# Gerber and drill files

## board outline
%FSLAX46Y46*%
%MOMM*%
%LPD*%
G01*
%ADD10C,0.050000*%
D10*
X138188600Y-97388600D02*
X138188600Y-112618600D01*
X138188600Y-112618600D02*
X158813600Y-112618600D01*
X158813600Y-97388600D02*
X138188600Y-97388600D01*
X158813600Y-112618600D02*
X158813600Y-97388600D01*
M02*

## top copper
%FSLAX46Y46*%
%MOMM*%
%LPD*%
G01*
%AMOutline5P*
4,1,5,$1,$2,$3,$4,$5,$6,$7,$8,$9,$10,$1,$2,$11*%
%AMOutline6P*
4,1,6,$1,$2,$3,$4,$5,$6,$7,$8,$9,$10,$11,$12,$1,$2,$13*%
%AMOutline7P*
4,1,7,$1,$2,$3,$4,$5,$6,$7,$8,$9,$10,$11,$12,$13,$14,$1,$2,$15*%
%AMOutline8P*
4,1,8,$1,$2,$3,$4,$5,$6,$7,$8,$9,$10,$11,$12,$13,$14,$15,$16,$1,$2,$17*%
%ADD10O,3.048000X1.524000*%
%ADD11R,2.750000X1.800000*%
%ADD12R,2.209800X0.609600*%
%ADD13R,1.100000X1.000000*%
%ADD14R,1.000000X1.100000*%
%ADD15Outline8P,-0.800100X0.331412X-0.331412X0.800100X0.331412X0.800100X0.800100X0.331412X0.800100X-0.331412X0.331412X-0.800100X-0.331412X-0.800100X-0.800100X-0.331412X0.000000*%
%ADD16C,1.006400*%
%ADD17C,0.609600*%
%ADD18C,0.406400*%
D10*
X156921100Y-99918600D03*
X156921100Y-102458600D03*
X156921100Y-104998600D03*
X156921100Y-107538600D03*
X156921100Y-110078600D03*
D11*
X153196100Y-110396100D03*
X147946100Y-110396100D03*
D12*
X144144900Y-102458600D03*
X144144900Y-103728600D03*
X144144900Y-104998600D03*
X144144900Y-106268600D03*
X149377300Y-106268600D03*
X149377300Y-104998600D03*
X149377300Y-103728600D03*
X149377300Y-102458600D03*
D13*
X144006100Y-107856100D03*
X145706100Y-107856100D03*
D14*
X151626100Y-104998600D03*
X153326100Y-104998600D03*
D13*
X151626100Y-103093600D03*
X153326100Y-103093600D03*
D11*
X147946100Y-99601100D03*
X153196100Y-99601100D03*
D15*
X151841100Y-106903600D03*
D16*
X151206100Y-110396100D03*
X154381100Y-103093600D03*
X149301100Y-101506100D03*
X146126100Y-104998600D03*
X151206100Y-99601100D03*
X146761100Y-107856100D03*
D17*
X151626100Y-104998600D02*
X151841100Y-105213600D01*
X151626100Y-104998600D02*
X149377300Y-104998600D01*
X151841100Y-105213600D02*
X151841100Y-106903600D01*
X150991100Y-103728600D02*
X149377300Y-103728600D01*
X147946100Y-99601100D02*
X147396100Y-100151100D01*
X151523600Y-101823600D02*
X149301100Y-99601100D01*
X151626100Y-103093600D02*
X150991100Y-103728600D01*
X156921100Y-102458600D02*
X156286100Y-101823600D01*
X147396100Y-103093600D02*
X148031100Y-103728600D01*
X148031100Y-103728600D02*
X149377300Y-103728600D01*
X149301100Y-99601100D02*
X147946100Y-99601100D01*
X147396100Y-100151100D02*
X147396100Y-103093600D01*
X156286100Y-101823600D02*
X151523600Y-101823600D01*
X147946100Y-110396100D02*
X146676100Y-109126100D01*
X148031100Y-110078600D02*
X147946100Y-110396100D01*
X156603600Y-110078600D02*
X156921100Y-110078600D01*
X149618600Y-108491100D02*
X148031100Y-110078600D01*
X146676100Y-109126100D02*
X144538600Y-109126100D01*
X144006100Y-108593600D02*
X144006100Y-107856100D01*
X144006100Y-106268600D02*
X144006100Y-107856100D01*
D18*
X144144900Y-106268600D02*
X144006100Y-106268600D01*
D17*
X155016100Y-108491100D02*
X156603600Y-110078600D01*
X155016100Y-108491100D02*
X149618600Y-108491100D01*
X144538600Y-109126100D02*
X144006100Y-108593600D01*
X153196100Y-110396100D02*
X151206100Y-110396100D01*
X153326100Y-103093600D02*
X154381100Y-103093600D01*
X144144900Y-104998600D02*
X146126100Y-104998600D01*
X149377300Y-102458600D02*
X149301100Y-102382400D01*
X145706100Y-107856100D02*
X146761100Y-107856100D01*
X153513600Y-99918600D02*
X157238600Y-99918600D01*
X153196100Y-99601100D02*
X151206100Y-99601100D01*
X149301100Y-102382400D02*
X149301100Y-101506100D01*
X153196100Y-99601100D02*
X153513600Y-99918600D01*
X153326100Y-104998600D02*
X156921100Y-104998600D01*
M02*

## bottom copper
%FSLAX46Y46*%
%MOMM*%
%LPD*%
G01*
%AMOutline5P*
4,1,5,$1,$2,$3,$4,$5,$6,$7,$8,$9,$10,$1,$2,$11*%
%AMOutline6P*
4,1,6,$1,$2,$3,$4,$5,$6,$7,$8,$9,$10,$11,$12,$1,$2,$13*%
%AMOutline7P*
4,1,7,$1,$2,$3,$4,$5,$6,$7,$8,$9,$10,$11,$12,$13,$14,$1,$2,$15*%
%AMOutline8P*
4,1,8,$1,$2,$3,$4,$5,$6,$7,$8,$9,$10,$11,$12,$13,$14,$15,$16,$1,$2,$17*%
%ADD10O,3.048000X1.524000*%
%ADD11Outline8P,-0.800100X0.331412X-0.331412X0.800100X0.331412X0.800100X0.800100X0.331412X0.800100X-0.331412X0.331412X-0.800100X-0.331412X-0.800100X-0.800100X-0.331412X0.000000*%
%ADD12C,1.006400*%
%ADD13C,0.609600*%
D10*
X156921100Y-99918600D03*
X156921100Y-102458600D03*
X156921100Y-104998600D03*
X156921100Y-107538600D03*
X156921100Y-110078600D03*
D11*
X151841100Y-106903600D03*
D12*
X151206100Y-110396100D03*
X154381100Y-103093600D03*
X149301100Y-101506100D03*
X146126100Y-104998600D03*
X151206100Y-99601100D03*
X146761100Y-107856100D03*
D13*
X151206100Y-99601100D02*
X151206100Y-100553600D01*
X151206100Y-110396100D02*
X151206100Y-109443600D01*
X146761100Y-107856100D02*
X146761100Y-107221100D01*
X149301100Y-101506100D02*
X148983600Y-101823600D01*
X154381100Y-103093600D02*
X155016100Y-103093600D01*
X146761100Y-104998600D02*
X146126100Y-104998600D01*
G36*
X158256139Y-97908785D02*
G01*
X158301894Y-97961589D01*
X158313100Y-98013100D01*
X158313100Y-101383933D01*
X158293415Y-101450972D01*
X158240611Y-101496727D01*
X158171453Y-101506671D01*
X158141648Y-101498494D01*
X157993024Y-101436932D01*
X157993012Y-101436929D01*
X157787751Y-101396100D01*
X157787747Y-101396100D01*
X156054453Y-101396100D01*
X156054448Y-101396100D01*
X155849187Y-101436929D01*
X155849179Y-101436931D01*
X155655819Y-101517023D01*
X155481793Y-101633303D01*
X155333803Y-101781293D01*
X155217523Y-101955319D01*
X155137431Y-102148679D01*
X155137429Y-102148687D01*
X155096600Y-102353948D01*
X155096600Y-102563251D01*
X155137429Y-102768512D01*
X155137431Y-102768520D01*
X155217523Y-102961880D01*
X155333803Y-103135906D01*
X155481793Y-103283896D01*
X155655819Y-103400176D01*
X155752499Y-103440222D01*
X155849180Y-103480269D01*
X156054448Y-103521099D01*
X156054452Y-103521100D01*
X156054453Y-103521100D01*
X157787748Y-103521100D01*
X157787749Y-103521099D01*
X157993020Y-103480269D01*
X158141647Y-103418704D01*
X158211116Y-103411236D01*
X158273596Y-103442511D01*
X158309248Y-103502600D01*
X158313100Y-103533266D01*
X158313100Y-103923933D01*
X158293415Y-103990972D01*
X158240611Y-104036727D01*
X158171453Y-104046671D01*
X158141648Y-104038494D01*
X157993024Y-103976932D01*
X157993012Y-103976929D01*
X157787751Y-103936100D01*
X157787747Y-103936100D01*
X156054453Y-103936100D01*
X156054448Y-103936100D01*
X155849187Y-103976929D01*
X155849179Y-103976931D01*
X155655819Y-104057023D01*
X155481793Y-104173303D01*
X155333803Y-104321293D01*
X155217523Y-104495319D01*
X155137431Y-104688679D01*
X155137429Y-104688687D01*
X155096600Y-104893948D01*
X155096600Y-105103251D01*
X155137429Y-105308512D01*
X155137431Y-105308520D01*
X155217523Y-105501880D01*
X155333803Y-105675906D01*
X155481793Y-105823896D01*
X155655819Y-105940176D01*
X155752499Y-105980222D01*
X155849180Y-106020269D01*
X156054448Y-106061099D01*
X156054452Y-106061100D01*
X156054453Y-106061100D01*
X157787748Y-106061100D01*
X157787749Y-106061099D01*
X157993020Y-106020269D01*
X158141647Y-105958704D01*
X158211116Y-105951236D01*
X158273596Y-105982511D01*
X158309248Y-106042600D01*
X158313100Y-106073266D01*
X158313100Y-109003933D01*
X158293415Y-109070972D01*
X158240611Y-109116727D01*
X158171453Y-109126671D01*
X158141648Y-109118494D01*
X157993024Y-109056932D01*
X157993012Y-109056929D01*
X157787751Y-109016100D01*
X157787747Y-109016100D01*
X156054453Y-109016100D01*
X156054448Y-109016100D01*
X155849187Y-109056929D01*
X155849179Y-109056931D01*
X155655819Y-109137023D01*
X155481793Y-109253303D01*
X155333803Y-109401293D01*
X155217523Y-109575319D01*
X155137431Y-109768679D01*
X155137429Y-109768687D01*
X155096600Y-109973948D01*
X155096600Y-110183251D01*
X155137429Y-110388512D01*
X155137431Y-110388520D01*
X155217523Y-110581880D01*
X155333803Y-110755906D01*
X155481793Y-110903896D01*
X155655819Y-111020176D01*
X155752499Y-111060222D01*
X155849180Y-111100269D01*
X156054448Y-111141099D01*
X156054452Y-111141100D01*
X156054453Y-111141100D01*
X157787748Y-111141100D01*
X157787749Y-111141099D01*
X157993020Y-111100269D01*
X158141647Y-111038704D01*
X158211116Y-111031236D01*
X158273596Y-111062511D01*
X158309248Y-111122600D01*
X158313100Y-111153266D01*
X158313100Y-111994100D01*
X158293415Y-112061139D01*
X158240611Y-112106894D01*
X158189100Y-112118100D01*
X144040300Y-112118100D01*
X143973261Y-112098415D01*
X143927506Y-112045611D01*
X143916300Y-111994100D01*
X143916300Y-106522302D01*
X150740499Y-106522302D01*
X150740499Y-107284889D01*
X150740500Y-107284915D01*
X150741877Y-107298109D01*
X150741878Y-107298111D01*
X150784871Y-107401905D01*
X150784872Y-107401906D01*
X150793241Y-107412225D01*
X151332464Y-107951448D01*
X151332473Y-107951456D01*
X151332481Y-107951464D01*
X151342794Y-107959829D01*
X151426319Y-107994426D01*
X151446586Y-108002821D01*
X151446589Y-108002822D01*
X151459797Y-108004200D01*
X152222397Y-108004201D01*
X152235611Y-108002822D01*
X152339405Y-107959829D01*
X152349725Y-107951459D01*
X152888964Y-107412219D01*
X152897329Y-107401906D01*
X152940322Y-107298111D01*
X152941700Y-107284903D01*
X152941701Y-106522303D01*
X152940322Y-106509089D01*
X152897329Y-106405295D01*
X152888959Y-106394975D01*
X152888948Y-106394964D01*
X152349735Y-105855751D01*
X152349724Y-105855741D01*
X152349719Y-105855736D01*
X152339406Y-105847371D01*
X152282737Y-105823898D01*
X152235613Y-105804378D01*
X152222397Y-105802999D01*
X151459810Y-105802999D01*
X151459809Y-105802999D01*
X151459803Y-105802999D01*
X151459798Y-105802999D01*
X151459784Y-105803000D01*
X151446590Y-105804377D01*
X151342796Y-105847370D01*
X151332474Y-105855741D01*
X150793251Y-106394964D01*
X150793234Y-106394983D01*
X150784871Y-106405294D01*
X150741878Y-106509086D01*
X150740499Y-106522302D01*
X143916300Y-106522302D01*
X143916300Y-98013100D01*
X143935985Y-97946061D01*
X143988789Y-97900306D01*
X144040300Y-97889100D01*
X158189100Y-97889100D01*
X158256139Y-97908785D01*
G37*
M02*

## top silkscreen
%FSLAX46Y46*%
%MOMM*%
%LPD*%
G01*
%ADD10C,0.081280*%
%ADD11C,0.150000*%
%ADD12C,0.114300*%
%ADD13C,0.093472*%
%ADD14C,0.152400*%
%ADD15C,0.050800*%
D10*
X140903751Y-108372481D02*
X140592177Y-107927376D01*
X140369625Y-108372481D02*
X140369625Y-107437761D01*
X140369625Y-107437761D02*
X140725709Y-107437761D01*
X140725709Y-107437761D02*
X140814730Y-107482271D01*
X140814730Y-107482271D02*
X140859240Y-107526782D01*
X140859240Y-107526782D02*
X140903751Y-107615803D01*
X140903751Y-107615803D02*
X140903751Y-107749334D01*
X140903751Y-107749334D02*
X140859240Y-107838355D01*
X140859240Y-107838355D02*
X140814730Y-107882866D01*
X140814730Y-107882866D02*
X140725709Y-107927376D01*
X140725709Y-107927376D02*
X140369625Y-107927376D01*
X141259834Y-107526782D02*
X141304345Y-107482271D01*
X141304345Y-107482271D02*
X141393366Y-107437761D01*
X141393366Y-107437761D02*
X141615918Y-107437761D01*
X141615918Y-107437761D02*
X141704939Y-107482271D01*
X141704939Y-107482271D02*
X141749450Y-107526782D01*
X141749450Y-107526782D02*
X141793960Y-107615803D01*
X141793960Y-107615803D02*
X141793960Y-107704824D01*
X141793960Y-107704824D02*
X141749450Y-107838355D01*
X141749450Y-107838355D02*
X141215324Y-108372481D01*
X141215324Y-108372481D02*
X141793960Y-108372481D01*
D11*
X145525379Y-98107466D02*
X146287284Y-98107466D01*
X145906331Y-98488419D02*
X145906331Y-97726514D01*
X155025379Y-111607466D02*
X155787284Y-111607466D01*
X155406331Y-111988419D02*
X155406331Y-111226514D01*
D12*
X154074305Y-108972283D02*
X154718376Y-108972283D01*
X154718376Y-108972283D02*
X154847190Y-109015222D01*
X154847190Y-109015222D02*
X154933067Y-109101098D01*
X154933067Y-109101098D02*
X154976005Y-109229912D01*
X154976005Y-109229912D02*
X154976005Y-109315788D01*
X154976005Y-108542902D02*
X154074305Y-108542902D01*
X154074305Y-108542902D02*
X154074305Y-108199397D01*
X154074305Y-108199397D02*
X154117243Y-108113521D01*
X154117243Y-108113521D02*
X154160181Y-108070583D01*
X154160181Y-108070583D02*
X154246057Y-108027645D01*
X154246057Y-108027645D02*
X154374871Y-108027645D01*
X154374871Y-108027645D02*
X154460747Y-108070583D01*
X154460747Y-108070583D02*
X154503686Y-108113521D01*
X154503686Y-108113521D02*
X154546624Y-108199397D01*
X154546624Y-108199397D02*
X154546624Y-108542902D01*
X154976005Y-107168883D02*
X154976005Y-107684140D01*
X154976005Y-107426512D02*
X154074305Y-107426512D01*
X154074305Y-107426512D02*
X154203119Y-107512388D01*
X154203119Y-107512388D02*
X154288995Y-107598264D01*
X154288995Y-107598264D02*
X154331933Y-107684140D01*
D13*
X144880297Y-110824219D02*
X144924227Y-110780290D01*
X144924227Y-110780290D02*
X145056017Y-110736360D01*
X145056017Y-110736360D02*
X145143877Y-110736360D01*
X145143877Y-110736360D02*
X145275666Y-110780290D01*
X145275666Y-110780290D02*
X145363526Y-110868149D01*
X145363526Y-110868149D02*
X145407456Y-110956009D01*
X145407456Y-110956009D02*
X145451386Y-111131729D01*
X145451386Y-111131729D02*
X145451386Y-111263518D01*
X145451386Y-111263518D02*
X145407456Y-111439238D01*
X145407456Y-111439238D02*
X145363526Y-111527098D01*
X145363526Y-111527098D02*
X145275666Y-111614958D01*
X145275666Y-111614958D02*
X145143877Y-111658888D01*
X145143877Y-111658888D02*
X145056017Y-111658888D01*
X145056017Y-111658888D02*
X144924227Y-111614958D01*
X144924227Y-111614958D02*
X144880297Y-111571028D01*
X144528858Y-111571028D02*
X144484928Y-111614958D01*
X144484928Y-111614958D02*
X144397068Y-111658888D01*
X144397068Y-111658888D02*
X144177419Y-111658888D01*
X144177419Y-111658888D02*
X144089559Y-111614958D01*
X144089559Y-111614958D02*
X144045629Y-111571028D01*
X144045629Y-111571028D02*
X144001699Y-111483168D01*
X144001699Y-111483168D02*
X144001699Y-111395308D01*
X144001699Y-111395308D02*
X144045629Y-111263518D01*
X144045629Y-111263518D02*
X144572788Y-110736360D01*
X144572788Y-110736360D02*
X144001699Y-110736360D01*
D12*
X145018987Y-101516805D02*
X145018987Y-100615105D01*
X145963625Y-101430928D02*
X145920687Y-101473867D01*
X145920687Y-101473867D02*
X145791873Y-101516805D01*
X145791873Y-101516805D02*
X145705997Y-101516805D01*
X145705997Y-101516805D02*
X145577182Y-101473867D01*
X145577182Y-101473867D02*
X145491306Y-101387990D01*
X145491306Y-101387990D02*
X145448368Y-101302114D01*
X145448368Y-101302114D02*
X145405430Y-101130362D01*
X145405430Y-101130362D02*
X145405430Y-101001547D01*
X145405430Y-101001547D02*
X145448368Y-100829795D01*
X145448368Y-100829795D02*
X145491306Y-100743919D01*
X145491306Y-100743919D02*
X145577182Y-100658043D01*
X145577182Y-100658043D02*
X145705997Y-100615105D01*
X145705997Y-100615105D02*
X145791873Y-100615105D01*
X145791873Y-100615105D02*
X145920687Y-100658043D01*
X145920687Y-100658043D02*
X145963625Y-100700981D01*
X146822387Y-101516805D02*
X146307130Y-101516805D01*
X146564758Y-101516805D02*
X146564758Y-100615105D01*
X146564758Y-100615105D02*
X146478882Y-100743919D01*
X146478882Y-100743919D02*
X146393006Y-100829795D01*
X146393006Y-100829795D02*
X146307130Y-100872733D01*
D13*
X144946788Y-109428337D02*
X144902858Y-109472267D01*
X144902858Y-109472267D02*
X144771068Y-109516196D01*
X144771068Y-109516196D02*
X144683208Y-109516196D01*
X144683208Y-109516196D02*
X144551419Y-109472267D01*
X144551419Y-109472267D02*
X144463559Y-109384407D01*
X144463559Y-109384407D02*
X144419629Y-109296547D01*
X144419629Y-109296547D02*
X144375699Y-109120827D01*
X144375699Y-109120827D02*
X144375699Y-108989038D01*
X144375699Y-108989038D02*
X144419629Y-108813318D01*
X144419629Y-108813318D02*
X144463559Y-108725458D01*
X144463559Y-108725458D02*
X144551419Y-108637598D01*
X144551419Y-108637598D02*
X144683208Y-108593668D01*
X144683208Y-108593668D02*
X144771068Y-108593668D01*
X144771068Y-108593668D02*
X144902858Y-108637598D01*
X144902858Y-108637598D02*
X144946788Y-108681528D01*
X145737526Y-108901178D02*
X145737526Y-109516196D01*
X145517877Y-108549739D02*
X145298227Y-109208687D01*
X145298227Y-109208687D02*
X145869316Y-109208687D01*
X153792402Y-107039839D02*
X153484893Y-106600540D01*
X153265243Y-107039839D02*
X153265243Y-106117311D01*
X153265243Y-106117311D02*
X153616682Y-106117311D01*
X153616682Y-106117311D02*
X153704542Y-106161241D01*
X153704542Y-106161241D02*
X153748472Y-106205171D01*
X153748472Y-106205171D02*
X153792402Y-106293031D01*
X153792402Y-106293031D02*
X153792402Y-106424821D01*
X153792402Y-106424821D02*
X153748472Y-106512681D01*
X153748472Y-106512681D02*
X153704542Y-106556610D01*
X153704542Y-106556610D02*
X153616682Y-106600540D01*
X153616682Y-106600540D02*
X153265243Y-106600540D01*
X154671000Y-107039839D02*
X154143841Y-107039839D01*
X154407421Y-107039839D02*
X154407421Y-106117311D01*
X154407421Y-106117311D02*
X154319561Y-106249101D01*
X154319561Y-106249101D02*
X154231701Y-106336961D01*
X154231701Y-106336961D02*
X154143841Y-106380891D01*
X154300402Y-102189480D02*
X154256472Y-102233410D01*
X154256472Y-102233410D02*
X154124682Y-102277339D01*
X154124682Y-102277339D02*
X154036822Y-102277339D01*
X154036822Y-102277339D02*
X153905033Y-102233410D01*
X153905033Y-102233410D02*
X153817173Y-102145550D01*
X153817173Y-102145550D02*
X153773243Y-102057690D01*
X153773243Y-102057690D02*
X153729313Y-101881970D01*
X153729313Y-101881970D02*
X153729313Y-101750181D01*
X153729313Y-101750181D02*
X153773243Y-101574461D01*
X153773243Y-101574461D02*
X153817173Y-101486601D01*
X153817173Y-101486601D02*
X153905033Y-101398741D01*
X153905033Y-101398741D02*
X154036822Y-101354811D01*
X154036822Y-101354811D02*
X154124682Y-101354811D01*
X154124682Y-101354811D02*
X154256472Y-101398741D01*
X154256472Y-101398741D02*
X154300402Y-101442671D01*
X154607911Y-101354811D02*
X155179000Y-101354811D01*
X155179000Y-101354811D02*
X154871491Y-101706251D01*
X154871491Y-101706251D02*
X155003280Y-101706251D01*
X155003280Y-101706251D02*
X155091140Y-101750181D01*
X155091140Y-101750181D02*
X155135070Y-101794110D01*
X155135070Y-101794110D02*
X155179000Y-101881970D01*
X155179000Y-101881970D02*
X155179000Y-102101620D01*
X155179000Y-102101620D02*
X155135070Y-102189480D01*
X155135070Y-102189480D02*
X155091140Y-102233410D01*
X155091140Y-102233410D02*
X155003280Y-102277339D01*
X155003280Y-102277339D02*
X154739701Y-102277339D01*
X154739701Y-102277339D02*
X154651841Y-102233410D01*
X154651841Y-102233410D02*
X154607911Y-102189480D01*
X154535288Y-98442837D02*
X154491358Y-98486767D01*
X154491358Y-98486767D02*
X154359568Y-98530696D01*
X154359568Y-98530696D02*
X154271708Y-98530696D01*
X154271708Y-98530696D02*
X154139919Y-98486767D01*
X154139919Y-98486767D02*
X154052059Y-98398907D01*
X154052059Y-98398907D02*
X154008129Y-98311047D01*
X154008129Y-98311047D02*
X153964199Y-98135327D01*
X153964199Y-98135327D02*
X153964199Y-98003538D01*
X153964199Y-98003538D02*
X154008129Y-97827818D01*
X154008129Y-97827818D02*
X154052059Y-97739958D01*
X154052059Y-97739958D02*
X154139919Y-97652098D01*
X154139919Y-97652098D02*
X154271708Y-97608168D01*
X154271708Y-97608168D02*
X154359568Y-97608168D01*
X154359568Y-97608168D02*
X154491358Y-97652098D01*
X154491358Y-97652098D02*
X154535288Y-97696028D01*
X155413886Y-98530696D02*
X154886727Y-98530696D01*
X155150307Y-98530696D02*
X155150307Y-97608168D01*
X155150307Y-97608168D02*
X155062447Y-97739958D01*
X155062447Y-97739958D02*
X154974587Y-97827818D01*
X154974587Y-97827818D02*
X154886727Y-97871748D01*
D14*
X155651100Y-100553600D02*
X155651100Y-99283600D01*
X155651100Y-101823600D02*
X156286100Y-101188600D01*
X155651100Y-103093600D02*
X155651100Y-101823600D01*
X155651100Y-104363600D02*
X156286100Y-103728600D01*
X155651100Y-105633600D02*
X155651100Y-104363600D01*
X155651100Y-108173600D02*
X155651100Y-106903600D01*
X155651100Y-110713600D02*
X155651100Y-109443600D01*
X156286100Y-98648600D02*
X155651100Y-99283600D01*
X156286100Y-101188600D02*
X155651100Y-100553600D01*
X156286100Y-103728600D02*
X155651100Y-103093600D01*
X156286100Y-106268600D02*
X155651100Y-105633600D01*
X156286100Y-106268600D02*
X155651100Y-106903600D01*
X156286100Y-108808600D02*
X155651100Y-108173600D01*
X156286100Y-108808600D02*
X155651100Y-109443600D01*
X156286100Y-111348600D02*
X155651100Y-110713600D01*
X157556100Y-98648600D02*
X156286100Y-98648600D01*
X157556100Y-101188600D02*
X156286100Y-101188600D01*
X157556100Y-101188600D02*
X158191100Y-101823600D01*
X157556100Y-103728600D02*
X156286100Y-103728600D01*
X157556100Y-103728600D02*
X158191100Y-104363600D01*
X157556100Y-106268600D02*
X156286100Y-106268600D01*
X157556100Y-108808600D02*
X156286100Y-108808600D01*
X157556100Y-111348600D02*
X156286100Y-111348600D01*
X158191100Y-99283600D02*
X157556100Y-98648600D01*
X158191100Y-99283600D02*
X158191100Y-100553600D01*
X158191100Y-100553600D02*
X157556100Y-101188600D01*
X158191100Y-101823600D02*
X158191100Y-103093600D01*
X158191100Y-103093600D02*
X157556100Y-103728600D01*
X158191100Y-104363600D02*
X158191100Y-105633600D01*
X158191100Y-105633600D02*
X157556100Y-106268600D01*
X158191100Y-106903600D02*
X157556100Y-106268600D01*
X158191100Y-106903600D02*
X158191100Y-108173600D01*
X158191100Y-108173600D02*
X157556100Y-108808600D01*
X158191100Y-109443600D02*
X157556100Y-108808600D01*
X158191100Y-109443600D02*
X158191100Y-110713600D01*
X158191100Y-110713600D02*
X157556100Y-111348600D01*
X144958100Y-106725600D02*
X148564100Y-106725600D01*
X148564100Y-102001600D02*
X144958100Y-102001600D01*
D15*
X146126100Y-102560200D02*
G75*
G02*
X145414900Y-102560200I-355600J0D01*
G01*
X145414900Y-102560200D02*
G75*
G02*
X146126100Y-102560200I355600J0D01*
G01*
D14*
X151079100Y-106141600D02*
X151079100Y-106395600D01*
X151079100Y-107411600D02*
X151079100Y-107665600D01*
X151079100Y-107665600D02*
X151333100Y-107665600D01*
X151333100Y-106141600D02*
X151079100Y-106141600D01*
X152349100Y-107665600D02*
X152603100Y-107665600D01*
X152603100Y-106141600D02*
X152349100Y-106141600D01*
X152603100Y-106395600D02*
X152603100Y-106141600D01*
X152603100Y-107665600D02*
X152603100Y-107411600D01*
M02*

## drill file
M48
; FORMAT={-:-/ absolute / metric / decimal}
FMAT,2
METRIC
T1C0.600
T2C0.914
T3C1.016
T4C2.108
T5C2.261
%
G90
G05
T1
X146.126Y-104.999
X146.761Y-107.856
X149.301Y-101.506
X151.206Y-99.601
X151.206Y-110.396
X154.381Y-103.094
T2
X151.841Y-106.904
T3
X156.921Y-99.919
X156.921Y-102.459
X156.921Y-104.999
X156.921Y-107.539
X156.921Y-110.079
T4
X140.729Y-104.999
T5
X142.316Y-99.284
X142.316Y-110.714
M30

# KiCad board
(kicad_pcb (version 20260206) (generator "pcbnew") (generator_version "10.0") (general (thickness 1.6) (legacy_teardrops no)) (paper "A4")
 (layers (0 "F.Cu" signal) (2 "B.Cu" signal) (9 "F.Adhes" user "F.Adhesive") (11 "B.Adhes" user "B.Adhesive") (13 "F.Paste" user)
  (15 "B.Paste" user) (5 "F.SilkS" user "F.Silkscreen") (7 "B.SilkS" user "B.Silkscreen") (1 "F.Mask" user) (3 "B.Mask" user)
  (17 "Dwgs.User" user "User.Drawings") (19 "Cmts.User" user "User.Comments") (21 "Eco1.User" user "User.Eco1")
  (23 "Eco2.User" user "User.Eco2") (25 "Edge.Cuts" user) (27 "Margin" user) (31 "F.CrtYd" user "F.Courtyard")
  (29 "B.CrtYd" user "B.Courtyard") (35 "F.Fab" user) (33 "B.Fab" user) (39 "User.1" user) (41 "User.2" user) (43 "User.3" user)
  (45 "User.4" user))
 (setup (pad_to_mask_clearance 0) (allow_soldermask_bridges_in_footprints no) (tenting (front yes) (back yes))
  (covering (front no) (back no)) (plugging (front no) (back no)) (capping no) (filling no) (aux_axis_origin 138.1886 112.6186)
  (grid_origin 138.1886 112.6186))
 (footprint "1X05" (layer "F.Cu") (at 156.9211 104.9986 -90)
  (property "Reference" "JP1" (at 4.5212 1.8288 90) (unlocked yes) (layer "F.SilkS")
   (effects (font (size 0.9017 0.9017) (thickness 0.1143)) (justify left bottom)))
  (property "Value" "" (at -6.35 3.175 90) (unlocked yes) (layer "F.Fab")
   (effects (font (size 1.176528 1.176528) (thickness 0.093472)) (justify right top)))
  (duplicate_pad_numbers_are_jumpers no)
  (fp_line (start -4.445 1.27) (end -5.715 1.27) (stroke (width 0.1524) (type solid)) (layer "F.SilkS"))
  (fp_line (start -3.175 1.27) (end -3.81 0.635) (stroke (width 0.1524) (type solid)) (layer "F.SilkS"))
  (fp_line (start -1.905 1.27) (end -3.175 1.27) (stroke (width 0.1524) (type solid)) (layer "F.SilkS"))
  (fp_line (start -0.635 1.27) (end -1.27 0.635) (stroke (width 0.1524) (type solid)) (layer "F.SilkS"))
  (fp_line (start 0.635 1.27) (end -0.635 1.27) (stroke (width 0.1524) (type solid)) (layer "F.SilkS"))
  (fp_line (start 3.175 1.27) (end 1.905 1.27) (stroke (width 0.1524) (type solid)) (layer "F.SilkS"))
  (fp_line (start 5.715 1.27) (end 4.445 1.27) (stroke (width 0.1524) (type solid)) (layer "F.SilkS"))
  (fp_line (start -6.35 0.635) (end -5.715 1.27) (stroke (width 0.1524) (type solid)) (layer "F.SilkS"))
  (fp_line (start -3.81 0.635) (end -4.445 1.27) (stroke (width 0.1524) (type solid)) (layer "F.SilkS"))
  (fp_line (start -1.27 0.635) (end -1.905 1.27) (stroke (width 0.1524) (type solid)) (layer "F.SilkS"))
  (fp_line (start 1.27 0.635) (end 0.635 1.27) (stroke (width 0.1524) (type solid)) (layer "F.SilkS"))
  (fp_line (start 1.27 0.635) (end 1.905 1.27) (stroke (width 0.1524) (type solid)) (layer "F.SilkS"))
  (fp_line (start 3.81 0.635) (end 3.175 1.27) (stroke (width 0.1524) (type solid)) (layer "F.SilkS"))
  (fp_line (start 3.81 0.635) (end 4.445 1.27) (stroke (width 0.1524) (type solid)) (layer "F.SilkS"))
  (fp_line (start 6.35 0.635) (end 5.715 1.27) (stroke (width 0.1524) (type solid)) (layer "F.SilkS"))
  (fp_line (start -6.35 -0.635) (end -6.35 0.635) (stroke (width 0.1524) (type solid)) (layer "F.SilkS"))
  (fp_line (start -3.81 -0.635) (end -3.81 0.635) (stroke (width 0.1524) (type solid)) (layer "F.SilkS"))
  (fp_line (start -3.81 -0.635) (end -3.175 -1.27) (stroke (width 0.1524) (type solid)) (layer "F.SilkS"))
  (fp_line (start -1.27 -0.635) (end -1.27 0.635) (stroke (width 0.1524) (type solid)) (layer "F.SilkS"))
  (fp_line (start -1.27 -0.635) (end -0.635 -1.27) (stroke (width 0.1524) (type solid)) (layer "F.SilkS"))
  (fp_line (start 1.27 -0.635) (end 1.27 0.635) (stroke (width 0.1524) (type solid)) (layer "F.SilkS"))
  (fp_line (start 3.81 -0.635) (end 3.81 0.635) (stroke (width 0.1524) (type solid)) (layer "F.SilkS"))
  (fp_line (start 6.35 -0.635) (end 6.35 0.635) (stroke (width 0.1524) (type solid)) (layer "F.SilkS"))
  (fp_line (start -5.715 -1.27) (end -6.35 -0.635) (stroke (width 0.1524) (type solid)) (layer "F.SilkS"))
  (fp_line (start -5.715 -1.27) (end -4.445 -1.27) (stroke (width 0.1524) (type solid)) (layer "F.SilkS"))
  (fp_line (start -4.445 -1.27) (end -3.81 -0.635) (stroke (width 0.1524) (type solid)) (layer "F.SilkS"))
  (fp_line (start -3.175 -1.27) (end -1.905 -1.27) (stroke (width 0.1524) (type solid)) (layer "F.SilkS"))
  (fp_line (start -1.905 -1.27) (end -1.27 -0.635) (stroke (width 0.1524) (type solid)) (layer "F.SilkS"))
  (fp_line (start -0.635 -1.27) (end 0.635 -1.27) (stroke (width 0.1524) (type solid)) (layer "F.SilkS"))
  (fp_line (start 0.635 -1.27) (end 1.27 -0.635) (stroke (width 0.1524) (type solid)) (layer "F.SilkS"))
  (fp_line (start 1.905 -1.27) (end 1.27 -0.635) (stroke (width 0.1524) (type solid)) (layer "F.SilkS"))
  (fp_line (start 1.905 -1.27) (end 3.175 -1.27) (stroke (width 0.1524) (type solid)) (layer "F.SilkS"))
  (fp_line (start 3.175 -1.27) (end 3.81 -0.635) (stroke (width 0.1524) (type solid)) (layer "F.SilkS"))
  (fp_line (start 4.445 -1.27) (end 3.81 -0.635) (stroke (width 0.1524) (type solid)) (layer "F.SilkS"))
  (fp_line (start 4.445 -1.27) (end 5.715 -1.27) (stroke (width 0.1524) (type solid)) (layer "F.SilkS"))
  (fp_line (start 5.715 -1.27) (end 6.35 -0.635) (stroke (width 0.1524) (type solid)) (layer "F.SilkS"))
  (pad "1" thru_hole oval (at -5.08 0) (size 3.048 1.524) (drill 1.016) (layers "*.Cu" "*.Mask") (remove_unused_layers no) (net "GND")
   (solder_mask_margin 0.1016) (zone_connect 2) (thermal_bridge_angle 0))
  (pad "2" thru_hole oval (at -2.54 0) (size 3.048 1.524) (drill 1.016) (layers "*.Cu" "*.Mask") (remove_unused_layers no) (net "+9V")
   (solder_mask_margin 0.1016) (thermal_bridge_angle 0))
  (pad "3" thru_hole oval (at 0 0) (size 3.048 1.524) (drill 1.016) (layers "*.Cu" "*.Mask") (remove_unused_layers no) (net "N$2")
   (solder_mask_margin 0.1016) (thermal_bridge_angle 0))
  (pad "4" thru_hole oval (at 2.54 0) (size 3.048 1.524) (drill 1.016) (layers "*.Cu" "*.Mask") (remove_unused_layers no) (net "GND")
   (solder_mask_margin 0.1016) (zone_connect 2) (thermal_bridge_angle 0))
  (pad "5" thru_hole oval (at 5.08 0) (size 3.048 1.524) (drill 1.016) (layers "*.Cu" "*.Mask") (remove_unused_layers no) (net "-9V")
   (solder_mask_margin 0.1016) (thermal_bridge_angle 0)))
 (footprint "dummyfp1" (layer "F.Cu") (at 142.3161 110.7136)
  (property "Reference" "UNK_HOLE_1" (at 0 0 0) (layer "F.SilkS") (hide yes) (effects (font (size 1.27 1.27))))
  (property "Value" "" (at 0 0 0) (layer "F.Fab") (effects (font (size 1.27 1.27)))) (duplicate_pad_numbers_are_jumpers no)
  (pad "" np_thru_hole circle (at 0 0) (size 2.2606 2.2606) (drill 2.2606) (layers "*.Cu" "*.Mask")))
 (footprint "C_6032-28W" (layer "F.Cu") (at 150.5711 110.3961)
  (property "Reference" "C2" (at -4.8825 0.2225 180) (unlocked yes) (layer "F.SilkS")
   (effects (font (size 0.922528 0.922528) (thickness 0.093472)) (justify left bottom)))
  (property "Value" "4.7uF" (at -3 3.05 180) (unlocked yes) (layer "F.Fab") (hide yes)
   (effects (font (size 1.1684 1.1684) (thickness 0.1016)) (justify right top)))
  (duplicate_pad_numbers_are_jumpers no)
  (pad "+" smd rect (at 2.625 0) (size 2.75 1.8) (layers "F.Cu" "F.Mask" "F.Paste") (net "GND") (solder_mask_margin 0.1016)
   (solder_paste_margin 0) (thermal_bridge_angle 0))
  (pad "-" smd rect (at -2.625 0) (size 2.75 1.8) (layers "F.Cu" "F.Mask" "F.Paste") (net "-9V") (solder_mask_margin 0.1016)
   (solder_paste_margin 0) (thermal_bridge_angle 0)))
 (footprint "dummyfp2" (layer "F.Cu") (at 142.3161 99.2836)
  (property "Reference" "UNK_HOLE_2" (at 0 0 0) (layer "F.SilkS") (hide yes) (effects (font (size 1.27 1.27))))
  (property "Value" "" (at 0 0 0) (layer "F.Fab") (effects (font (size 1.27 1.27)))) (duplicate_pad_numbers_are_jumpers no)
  (pad "" np_thru_hole circle (at 0 0) (size 2.2606 2.2606) (drill 2.2606) (layers "*.Cu" "*.Mask")))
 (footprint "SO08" (layer "F.Cu") (at 146.7611 104.3636 -90)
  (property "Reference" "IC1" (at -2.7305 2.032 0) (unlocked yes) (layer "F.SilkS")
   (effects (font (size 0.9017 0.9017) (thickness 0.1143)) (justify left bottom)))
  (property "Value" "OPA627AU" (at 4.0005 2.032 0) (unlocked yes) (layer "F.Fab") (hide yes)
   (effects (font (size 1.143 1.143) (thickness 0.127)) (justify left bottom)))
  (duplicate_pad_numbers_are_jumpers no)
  (fp_line (start 2.362 1.803) (end 2.362 -1.803) (stroke (width 0.1524) (type solid)) (layer "F.SilkS"))
  (fp_line (start -2.362 -1.803) (end -2.362 1.803) (stroke (width 0.1524) (type solid)) (layer "F.SilkS"))
  (fp_circle (center -1.8034 0.9906) (end -1.4478 0.9906) (stroke (width 0.0508) (type solid)) (fill no) (layer "F.SilkS"))
  (pad "1" smd rect (at -1.905 2.6162 270) (size 0.6096 2.2098) (layers "F.Cu" "F.Mask" "F.Paste") (solder_mask_margin 0.1016)
   (solder_paste_margin 0) (thermal_bridge_angle 0))
  (pad "2" smd rect (at -0.635 2.6162 270) (size 0.6096 2.2098) (layers "F.Cu" "F.Mask" "F.Paste") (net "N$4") (solder_mask_margin 0.1016)
   (solder_paste_margin 0) (thermal_bridge_angle 0))
  (pad "3" smd rect (at 0.635 2.6162 270) (size 0.6096 2.2098) (layers "F.Cu" "F.Mask" "F.Paste") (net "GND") (solder_mask_margin 0.1016)
   (solder_paste_margin 0) (thermal_bridge_angle 0))
  (pad "4" smd rect (at 1.905 2.6162 270) (size 0.6096 2.2098) (layers "F.Cu" "F.Mask" "F.Paste") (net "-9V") (solder_mask_margin 0.1016)
   (solder_paste_margin 0) (thermal_bridge_angle 0))
  (pad "5" smd rect (at 1.905 -2.6162 270) (size 0.6096 2.2098) (layers "F.Cu" "F.Mask" "F.Paste") (solder_mask_margin 0.1016)
   (solder_paste_margin 0) (thermal_bridge_angle 0))
  (pad "6" smd rect (at 0.635 -2.6162 270) (size 0.6096 2.2098) (layers "F.Cu" "F.Mask" "F.Paste") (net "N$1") (solder_mask_margin 0.1016)
   (solder_paste_margin 0) (thermal_bridge_angle 0))
  (pad "7" smd rect (at -0.635 -2.6162 270) (size 0.6096 2.2098) (layers "F.Cu" "F.Mask" "F.Paste") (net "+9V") (solder_mask_margin 0.1016)
   (solder_paste_margin 0) (thermal_bridge_angle 0))
  (pad "8" smd rect (at -1.905 -2.6162 270) (size 0.6096 2.2098) (layers "F.Cu" "F.Mask" "F.Paste") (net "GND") (solder_mask_margin 0.1016)
   (solder_paste_margin 0) (thermal_bridge_angle 0)))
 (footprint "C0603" (layer "F.Cu") (at 144.8561 107.8561)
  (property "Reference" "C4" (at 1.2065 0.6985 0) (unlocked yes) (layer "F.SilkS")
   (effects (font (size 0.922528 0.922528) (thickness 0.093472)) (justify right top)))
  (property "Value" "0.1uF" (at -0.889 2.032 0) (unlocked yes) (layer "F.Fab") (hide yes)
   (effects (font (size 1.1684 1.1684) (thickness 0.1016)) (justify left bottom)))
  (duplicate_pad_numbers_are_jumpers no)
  (pad "1" smd rect (at -0.85 0) (size 1.1 1) (layers "F.Cu" "F.Mask" "F.Paste") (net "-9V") (solder_mask_margin 0.1016)
   (solder_paste_margin 0) (thermal_bridge_angle 0))
  (pad "2" smd rect (at 0.85 0) (size 1.1 1) (layers "F.Cu" "F.Mask" "F.Paste") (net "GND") (solder_mask_margin 0.1016)
   (solder_paste_margin 0) (thermal_bridge_angle 0)))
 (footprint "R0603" (layer "F.Cu") (at 152.4761 104.9986)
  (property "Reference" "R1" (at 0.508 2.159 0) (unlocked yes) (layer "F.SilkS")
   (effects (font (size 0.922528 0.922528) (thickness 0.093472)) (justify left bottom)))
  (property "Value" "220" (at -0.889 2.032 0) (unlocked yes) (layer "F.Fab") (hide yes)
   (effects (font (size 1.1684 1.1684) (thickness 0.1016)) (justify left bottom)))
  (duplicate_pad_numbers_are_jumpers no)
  (pad "1" smd rect (at -0.85 0) (size 1 1.1) (layers "F.Cu" "F.Mask" "F.Paste") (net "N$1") (solder_mask_margin 0.1016)
   (solder_paste_margin 0) (thermal_bridge_angle 0))
  (pad "2" smd rect (at 0.85 0) (size 1 1.1) (layers "F.Cu" "F.Mask" "F.Paste") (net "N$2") (solder_mask_margin 0.1016)
   (solder_paste_margin 0) (thermal_bridge_angle 0)))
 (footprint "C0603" (layer "F.Cu") (at 152.4761 103.0936)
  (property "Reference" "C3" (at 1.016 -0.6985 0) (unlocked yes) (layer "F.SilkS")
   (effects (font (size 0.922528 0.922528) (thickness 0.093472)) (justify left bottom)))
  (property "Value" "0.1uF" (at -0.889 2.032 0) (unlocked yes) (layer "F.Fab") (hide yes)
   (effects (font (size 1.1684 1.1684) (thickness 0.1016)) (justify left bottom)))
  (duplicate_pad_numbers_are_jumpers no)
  (pad "1" smd rect (at -0.85 0) (size 1.1 1) (layers "F.Cu" "F.Mask" "F.Paste") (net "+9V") (solder_mask_margin 0.1016)
   (solder_paste_margin 0) (thermal_bridge_angle 0))
  (pad "2" smd rect (at 0.85 0) (size 1.1 1) (layers "F.Cu" "F.Mask" "F.Paste") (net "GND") (solder_mask_margin 0.1016)
   (solder_paste_margin 0) (thermal_bridge_angle 0)))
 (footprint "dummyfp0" (layer "F.Cu") (at 140.7286 104.9986)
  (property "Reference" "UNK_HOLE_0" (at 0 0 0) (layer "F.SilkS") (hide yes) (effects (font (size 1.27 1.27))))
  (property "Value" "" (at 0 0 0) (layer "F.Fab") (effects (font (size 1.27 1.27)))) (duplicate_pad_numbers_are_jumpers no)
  (pad "" np_thru_hole circle (at 0 0) (size 2.1082 2.1082) (drill 2.1082) (layers "*.Cu" "*.Mask")))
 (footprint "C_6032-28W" (layer "F.Cu") (at 150.5711 99.6011 180)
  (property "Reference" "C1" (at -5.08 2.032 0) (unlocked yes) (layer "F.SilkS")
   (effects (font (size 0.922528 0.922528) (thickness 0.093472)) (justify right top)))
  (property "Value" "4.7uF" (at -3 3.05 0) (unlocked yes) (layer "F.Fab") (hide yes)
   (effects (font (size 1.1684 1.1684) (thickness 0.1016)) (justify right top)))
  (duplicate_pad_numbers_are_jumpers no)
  (pad "+" smd rect (at 2.625 0 180) (size 2.75 1.8) (layers "F.Cu" "F.Mask" "F.Paste") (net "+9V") (solder_mask_margin 0.1016)
   (solder_paste_margin 0) (thermal_bridge_angle 0))
  (pad "-" smd rect (at -2.625 0 180) (size 2.75 1.8) (layers "F.Cu" "F.Mask" "F.Paste") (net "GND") (solder_mask_margin 0.1016)
   (solder_paste_margin 0) (thermal_bridge_angle 0)))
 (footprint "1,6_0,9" (layer "F.Cu") (at 151.8411 106.9036)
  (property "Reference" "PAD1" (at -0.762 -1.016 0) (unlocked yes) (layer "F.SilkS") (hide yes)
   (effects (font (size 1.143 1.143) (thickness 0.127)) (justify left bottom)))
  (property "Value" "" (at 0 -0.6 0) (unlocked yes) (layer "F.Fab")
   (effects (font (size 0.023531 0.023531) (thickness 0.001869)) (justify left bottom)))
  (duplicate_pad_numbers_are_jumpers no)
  (fp_line (start -0.762 -0.762) (end -0.762 -0.508) (stroke (width 0.1524) (type solid)) (layer "F.SilkS"))
  (fp_line (start -0.762 0.508) (end -0.762 0.762) (stroke (width 0.1524) (type solid)) (layer "F.SilkS"))
  (fp_line (start -0.762 0.762) (end -0.508 0.762) (stroke (width 0.1524) (type solid)) (layer "F.SilkS"))
  (fp_line (start -0.508 -0.762) (end -0.762 -0.762) (stroke (width 0.1524) (type solid)) (layer "F.SilkS"))
  (fp_line (start 0.508 0.762) (end 0.762 0.762) (stroke (width 0.1524) (type solid)) (layer "F.SilkS"))
  (fp_line (start 0.762 -0.762) (end 0.508 -0.762) (stroke (width 0.1524) (type solid)) (layer "F.SilkS"))
  (fp_line (start 0.762 -0.508) (end 0.762 -0.762) (stroke (width 0.1524) (type solid)) (layer "F.SilkS"))
  (fp_line (start 0.762 0.762) (end 0.762 0.508) (stroke (width 0.1524) (type solid)) (layer "F.SilkS"))
  (pad "1" thru_hole roundrect (at 0 0) (size 1.6002 1.6002) (drill 0.9144) (layers "*.Cu" "*.Mask") (remove_unused_layers no)
   (roundrect_rratio 0.25) (chamfer_ratio 0.2928932188) (chamfer top_left top_right bottom_left bottom_right) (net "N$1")
   (solder_mask_margin 0.1016) (thermal_bridge_angle 0)))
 (gr_line (start 138.1886 97.3886) (end 138.1886 112.6186) (stroke (width 0.05) (type solid)) (layer "Edge.Cuts"))
 (gr_line (start 138.1886 112.6186) (end 158.8136 112.6186) (stroke (width 0.05) (type solid)) (layer "Edge.Cuts"))
 (gr_line (start 158.8136 97.3886) (end 138.1886 97.3886) (stroke (width 0.05) (type solid)) (layer "Edge.Cuts"))
 (gr_line (start 158.8136 112.6186) (end 158.8136 97.3886) (stroke (width 0.05) (type solid)) (layer "Edge.Cuts"))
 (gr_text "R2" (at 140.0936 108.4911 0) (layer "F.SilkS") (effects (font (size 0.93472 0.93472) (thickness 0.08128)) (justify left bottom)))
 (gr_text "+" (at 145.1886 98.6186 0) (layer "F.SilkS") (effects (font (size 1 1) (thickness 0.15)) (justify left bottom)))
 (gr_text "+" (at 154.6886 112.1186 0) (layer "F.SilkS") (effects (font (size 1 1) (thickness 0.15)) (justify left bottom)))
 (segment (start 151.6261 104.9986) (end 151.8411 105.2136) (width 0.6096) (layer "F.Cu") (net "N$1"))
 (segment (start 151.6261 104.9986) (end 149.3773 104.9986) (width 0.6096) (layer "F.Cu") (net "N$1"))
 (segment (start 151.8411 105.2136) (end 151.8411 106.9036) (width 0.6096) (layer "F.Cu") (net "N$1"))
 (segment (start 150.9911 103.7286) (end 149.3773 103.7286) (width 0.6096) (layer "F.Cu") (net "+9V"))
 (segment (start 147.9461 99.6011) (end 147.3961 100.1511) (width 0.6096) (layer "F.Cu") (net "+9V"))
 (segment (start 151.5236 101.8236) (end 149.3011 99.6011) (width 0.6096) (layer "F.Cu") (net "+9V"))
 (segment (start 151.6261 103.0936) (end 150.9911 103.7286) (width 0.6096) (layer "F.Cu") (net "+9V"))
 (segment (start 156.9211 102.4586) (end 156.2861 101.8236) (width 0.6096) (layer "F.Cu") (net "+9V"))
 (segment (start 147.3961 103.0936) (end 148.0311 103.7286) (width 0.6096) (layer "F.Cu") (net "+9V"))
 (segment (start 148.0311 103.7286) (end 149.3773 103.7286) (width 0.6096) (layer "F.Cu") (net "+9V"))
 (segment (start 149.3011 99.6011) (end 147.9461 99.6011) (width 0.6096) (layer "F.Cu") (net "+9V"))
 (segment (start 147.3961 100.1511) (end 147.3961 103.0936) (width 0.6096) (layer "F.Cu") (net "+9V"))
 (segment (start 156.2861 101.8236) (end 151.5236 101.8236) (width 0.6096) (layer "F.Cu") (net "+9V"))
 (segment (start 147.9461 110.3961) (end 146.6761 109.1261) (width 0.6096) (layer "F.Cu") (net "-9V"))
 (segment (start 148.0311 110.0786) (end 147.9461 110.3961) (width 0.6096) (layer "F.Cu") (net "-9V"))
 (segment (start 156.6036 110.0786) (end 156.9211 110.0786) (width 0.6096) (layer "F.Cu") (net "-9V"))
 (segment (start 149.6186 108.4911) (end 148.0311 110.0786) (width 0.6096) (layer "F.Cu") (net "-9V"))
 (segment (start 146.6761 109.1261) (end 144.5386 109.1261) (width 0.6096) (layer "F.Cu") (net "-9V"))
 (segment (start 144.0061 108.5936) (end 144.0061 107.8561) (width 0.6096) (layer "F.Cu") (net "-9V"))
 (segment (start 144.0061 106.2686) (end 144.0061 107.8561) (width 0.6096) (layer "F.Cu") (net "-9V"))
 (segment (start 144.1449 106.2686) (end 144.0061 106.2686) (width 0.4064) (layer "F.Cu") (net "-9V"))
 (segment (start 155.0161 108.4911) (end 156.6036 110.0786) (width 0.6096) (layer "F.Cu") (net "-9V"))
 (segment (start 155.0161 108.4911) (end 149.6186 108.4911) (width 0.6096) (layer "F.Cu") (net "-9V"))
 (segment (start 144.5386 109.1261) (end 144.0061 108.5936) (width 0.6096) (layer "F.Cu") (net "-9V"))
 (segment (start 153.1961 110.3961) (end 151.2061 110.3961) (width 0.6096) (layer "F.Cu") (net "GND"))
 (segment (start 153.3261 103.0936) (end 154.3811 103.0936) (width 0.6096) (layer "F.Cu") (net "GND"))
 (segment (start 144.1449 104.9986) (end 146.1261 104.9986) (width 0.6096) (layer "F.Cu") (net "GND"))
 (segment (start 149.3773 102.4586) (end 149.3011 102.3824) (width 0.6096) (layer "F.Cu") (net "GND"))
 (segment (start 145.7061 107.8561) (end 146.7611 107.8561) (width 0.6096) (layer "F.Cu") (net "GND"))
 (segment (start 153.5136 99.9186) (end 157.2386 99.9186) (width 0.6096) (layer "F.Cu") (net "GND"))
 (segment (start 153.1961 99.6011) (end 151.2061 99.6011) (width 0.6096) (layer "F.Cu") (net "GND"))
 (segment (start 149.3011 102.3824) (end 149.3011 101.5061) (width 0.6096) (layer "F.Cu") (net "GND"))
 (segment (start 153.1961 99.6011) (end 153.5136 99.9186) (width 0.6096) (layer "F.Cu") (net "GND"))
 (via (at 151.2061 110.3961) (size 1.0064) (drill 0.6) (layers "F.Cu" "B.Cu") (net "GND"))
 (via (at 154.3811 103.0936) (size 1.0064) (drill 0.6) (layers "F.Cu" "B.Cu") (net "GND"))
 (via (at 149.3011 101.5061) (size 1.0064) (drill 0.6) (layers "F.Cu" "B.Cu") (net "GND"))
 (via (at 146.1261 104.9986) (size 1.0064) (drill 0.6) (layers "F.Cu" "B.Cu") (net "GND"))
 (via (at 151.2061 99.6011) (size 1.0064) (drill 0.6) (layers "F.Cu" "B.Cu") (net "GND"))
 (via (at 146.7611 107.8561) (size 1.0064) (drill 0.6) (layers "F.Cu" "B.Cu") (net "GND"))
 (segment (start 151.2061 99.6011) (end 151.2061 100.5536) (width 0.6096) (layer "B.Cu") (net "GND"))
 (segment (start 151.2061 110.3961) (end 151.2061 109.4436) (width 0.6096) (layer "B.Cu") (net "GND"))
 (segment (start 146.7611 107.8561) (end 146.7611 107.2211) (width 0.6096) (layer "B.Cu") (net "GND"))
 (segment (start 149.3011 101.5061) (end 148.9836 101.8236) (width 0.6096) (layer "B.Cu") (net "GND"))
 (segment (start 154.3811 103.0936) (end 155.0161 103.0936) (width 0.6096) (layer "B.Cu") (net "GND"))
 (segment (start 146.7611 104.9986) (end 146.1261 104.9986) (width 0.6096) (layer "B.Cu") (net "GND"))
 (segment (start 153.3261 104.9986) (end 156.9211 104.9986) (width 0.6096) (layer "F.Cu") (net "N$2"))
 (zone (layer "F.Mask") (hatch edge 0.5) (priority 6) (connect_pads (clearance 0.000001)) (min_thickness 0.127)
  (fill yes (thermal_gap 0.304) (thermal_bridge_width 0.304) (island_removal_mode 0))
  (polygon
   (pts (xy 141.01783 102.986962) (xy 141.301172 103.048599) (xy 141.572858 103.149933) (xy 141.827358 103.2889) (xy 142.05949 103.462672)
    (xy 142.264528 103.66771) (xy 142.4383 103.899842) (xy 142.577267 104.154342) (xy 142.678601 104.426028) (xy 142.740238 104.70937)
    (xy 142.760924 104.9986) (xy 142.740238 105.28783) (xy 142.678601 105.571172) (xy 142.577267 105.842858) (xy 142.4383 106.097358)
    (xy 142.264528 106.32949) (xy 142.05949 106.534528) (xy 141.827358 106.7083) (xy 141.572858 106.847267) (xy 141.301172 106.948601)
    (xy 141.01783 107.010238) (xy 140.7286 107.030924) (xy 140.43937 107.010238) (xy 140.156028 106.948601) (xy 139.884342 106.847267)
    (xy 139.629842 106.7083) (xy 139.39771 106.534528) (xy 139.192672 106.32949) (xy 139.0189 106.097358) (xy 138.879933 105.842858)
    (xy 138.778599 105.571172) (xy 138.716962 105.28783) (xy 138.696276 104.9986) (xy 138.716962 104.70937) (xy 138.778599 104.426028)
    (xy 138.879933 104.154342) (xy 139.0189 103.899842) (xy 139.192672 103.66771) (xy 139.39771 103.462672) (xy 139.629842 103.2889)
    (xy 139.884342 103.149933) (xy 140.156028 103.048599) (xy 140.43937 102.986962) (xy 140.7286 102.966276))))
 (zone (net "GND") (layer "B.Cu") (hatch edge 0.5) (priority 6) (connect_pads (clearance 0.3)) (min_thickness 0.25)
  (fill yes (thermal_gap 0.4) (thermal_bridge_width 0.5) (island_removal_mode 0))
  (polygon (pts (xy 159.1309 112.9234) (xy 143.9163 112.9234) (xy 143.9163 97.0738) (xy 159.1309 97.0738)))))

